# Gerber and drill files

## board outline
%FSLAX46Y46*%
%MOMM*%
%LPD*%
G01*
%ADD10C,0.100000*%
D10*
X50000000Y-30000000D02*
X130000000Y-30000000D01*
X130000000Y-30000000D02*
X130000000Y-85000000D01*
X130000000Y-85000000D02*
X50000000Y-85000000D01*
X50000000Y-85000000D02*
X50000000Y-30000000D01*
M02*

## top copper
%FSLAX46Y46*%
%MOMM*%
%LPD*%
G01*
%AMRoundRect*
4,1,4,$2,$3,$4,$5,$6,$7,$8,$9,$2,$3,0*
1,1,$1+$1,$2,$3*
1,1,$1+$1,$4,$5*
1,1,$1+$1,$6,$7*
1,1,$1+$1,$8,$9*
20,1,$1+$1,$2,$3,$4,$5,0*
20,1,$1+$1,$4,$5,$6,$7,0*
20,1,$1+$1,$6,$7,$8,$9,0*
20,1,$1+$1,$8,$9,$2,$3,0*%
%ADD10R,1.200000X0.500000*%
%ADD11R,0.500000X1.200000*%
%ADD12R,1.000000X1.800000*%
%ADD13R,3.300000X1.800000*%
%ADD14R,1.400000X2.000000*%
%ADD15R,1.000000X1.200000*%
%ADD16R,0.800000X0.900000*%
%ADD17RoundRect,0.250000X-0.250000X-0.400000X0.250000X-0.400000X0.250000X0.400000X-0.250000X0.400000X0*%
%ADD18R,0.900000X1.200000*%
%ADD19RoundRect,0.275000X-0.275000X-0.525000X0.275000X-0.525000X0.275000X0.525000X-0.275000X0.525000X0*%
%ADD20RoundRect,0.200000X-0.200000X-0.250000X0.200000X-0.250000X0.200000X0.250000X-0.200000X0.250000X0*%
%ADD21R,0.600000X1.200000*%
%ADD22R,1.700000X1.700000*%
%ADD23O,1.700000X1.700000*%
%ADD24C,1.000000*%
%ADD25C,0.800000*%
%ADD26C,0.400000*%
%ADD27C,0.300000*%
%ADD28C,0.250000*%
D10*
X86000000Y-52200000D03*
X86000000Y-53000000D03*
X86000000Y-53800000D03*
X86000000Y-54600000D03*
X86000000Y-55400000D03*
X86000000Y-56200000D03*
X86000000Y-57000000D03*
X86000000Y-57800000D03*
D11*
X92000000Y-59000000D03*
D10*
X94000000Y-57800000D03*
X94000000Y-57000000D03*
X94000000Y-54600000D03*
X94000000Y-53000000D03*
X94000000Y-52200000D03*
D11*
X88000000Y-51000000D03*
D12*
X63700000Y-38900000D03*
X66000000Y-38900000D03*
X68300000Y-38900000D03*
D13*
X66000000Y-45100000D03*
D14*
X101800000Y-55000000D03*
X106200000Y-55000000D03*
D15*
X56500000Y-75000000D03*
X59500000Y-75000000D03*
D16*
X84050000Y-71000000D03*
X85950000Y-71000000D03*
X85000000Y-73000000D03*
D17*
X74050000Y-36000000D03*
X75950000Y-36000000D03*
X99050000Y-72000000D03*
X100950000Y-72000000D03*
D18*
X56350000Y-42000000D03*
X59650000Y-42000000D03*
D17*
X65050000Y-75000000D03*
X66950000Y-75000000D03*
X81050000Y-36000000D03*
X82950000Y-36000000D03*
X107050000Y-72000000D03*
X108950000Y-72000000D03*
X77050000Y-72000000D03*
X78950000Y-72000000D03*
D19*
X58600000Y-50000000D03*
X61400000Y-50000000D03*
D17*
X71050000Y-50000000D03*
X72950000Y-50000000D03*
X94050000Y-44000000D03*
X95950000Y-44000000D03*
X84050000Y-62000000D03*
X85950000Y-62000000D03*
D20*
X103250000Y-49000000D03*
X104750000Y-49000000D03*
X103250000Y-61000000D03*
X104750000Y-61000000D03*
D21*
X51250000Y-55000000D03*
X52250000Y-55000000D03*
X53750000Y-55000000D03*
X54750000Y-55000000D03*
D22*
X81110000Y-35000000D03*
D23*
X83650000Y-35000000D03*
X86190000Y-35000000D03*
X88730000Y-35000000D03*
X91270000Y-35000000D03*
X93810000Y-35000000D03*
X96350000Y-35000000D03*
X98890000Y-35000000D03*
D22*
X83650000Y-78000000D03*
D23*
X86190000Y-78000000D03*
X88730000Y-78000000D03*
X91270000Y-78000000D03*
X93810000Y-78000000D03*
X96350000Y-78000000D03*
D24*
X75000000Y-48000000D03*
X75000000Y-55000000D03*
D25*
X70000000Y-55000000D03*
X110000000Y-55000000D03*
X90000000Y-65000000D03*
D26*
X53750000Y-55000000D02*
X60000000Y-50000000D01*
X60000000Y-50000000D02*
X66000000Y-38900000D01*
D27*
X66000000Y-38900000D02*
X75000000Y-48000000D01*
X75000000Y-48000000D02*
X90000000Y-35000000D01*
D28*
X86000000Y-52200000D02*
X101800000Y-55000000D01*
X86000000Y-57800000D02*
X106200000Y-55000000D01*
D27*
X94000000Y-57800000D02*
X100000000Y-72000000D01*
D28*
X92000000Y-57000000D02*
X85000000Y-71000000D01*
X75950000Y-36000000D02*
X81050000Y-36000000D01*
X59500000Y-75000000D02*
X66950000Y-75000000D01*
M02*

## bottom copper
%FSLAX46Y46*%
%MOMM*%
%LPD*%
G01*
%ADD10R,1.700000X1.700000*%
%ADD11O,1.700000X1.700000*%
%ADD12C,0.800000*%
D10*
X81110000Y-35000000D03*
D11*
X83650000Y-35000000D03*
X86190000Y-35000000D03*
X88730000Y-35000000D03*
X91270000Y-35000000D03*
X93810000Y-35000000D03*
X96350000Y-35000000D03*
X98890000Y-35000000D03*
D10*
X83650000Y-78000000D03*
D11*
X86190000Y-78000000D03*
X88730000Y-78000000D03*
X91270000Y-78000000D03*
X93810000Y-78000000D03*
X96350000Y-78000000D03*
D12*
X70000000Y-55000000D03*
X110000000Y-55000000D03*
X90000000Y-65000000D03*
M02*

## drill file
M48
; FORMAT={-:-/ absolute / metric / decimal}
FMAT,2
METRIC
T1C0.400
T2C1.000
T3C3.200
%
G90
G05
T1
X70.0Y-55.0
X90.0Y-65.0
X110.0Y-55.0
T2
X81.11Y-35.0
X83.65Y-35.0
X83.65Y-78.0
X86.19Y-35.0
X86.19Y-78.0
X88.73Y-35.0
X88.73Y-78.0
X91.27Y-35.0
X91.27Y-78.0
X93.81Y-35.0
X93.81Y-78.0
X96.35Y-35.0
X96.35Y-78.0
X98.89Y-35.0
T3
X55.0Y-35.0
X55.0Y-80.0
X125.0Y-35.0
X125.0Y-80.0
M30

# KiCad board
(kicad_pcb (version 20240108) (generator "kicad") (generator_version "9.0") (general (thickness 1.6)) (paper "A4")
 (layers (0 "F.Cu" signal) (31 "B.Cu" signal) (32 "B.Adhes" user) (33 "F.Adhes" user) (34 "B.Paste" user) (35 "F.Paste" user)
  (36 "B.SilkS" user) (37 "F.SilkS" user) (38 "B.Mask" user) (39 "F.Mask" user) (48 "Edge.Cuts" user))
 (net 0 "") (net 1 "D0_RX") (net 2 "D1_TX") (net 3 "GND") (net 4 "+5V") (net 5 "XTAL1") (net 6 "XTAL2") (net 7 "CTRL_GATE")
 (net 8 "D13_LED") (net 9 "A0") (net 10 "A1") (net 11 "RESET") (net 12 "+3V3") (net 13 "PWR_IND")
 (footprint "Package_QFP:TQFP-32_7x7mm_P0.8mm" (layer "F.Cu") (at 90.0 55.0) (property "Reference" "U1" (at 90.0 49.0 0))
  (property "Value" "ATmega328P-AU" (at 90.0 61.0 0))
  (pad "1" smd rect (at -4.0 -2.8) (size 1.2 0.5) (layers "F.Cu" "F.Mask") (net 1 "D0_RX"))
  (pad "2" smd rect (at -4.0 -2.0) (size 1.2 0.5) (layers "F.Cu" "F.Mask") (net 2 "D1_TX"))
  (pad "3" smd rect (at -4.0 -1.2) (size 1.2 0.5) (layers "F.Cu" "F.Mask") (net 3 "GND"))
  (pad "4" smd rect (at -4.0 -0.4) (size 1.2 0.5) (layers "F.Cu" "F.Mask") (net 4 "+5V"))
  (pad "5" smd rect (at -4.0 0.4) (size 1.2 0.5) (layers "F.Cu" "F.Mask") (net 3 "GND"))
  (pad "6" smd rect (at -4.0 1.2) (size 1.2 0.5) (layers "F.Cu" "F.Mask") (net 4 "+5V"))
  (pad "7" smd rect (at -4.0 2.0) (size 1.2 0.5) (layers "F.Cu" "F.Mask") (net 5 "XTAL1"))
  (pad "8" smd rect (at -4.0 2.8) (size 1.2 0.5) (layers "F.Cu" "F.Mask") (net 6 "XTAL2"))
  (pad "15" smd rect (at 2.0 4.0) (size 0.5 1.2) (layers "F.Cu" "F.Mask") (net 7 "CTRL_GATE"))
  (pad "17" smd rect (at 4.0 2.8) (size 1.2 0.5) (layers "F.Cu" "F.Mask") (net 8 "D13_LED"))
  (pad "18" smd rect (at 4.0 2.0) (size 1.2 0.5) (layers "F.Cu" "F.Mask") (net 4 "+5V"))
  (pad "21" smd rect (at 4.0 -0.4) (size 1.2 0.5) (layers "F.Cu" "F.Mask") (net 3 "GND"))
  (pad "23" smd rect (at 4.0 -2.0) (size 1.2 0.5) (layers "F.Cu" "F.Mask") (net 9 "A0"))
  (pad "24" smd rect (at 4.0 -2.8) (size 1.2 0.5) (layers "F.Cu" "F.Mask") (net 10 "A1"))
  (pad "29" smd rect (at -2.0 -4.0) (size 0.5 1.2) (layers "F.Cu" "F.Mask") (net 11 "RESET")))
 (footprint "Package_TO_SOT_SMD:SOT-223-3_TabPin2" (layer "F.Cu") (at 66.0 42.0) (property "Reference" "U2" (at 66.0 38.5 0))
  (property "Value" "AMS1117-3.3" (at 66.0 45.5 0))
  (pad "1" smd rect (at -2.3 -3.1) (size 1.0 1.8) (layers "F.Cu" "F.Mask") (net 3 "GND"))
  (pad "2" smd rect (at 0.0 -3.1) (size 1.0 1.8) (layers "F.Cu" "F.Mask") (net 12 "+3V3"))
  (pad "3" smd rect (at 2.3 -3.1) (size 1.0 1.8) (layers "F.Cu" "F.Mask") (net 4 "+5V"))
  (pad "4" smd rect (at 0.0 3.1) (size 3.3 1.8) (layers "F.Cu" "F.Mask") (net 12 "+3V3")))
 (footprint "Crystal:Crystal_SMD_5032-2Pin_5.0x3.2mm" (layer "F.Cu") (at 104.0 55.0) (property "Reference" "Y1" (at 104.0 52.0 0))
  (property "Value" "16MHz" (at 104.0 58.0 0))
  (pad "1" smd rect (at -2.2 0) (size 1.4 2.0) (layers "F.Cu" "F.Mask") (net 5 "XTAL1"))
  (pad "2" smd rect (at 2.2 0) (size 1.4 2.0) (layers "F.Cu" "F.Mask") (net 6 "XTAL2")))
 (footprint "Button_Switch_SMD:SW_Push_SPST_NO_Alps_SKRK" (layer "F.Cu") (at 58.0 75.0) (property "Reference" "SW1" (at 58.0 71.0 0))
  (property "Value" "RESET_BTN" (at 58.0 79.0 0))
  (pad "1" smd rect (at -1.5 0) (size 1.0 1.2) (layers "F.Cu" "F.Mask") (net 11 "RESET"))
  (pad "2" smd rect (at 1.5 0) (size 1.0 1.2) (layers "F.Cu" "F.Mask") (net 3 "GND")))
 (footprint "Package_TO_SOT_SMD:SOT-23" (layer "F.Cu") (at 85.0 72.0) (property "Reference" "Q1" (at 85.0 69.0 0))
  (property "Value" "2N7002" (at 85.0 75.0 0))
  (pad "1" smd rect (at -0.95 -1.0) (size 0.8 0.9) (layers "F.Cu" "F.Mask") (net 7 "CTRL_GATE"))
  (pad "2" smd rect (at 0.95 -1.0) (size 0.8 0.9) (layers "F.Cu" "F.Mask") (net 3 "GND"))
  (pad "3" smd rect (at 0.0 1.0) (size 0.8 0.9) (layers "F.Cu" "F.Mask") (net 8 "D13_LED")))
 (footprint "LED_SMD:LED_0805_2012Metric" (layer "F.Cu") (at 75.0 36.0) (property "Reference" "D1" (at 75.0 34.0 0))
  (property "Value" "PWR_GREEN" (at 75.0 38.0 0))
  (pad "1" smd roundrect (at -0.95 0) (size 1.0 1.3) (layers "F.Cu" "F.Mask") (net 3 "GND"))
  (pad "2" smd roundrect (at 0.95 0) (size 1.0 1.3) (layers "F.Cu" "F.Mask") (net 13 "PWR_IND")))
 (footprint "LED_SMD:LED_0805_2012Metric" (layer "F.Cu") (at 100.0 72.0) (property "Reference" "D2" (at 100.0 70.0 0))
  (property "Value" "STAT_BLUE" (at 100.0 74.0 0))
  (pad "1" smd roundrect (at -0.95 0) (size 1.0 1.3) (layers "F.Cu" "F.Mask") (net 3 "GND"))
  (pad "2" smd roundrect (at 0.95 0) (size 1.0 1.3) (layers "F.Cu" "F.Mask") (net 8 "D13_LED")))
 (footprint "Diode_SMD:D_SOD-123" (layer "F.Cu") (at 58.0 42.0) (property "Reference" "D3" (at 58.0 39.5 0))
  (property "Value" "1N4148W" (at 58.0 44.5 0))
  (pad "1" smd rect (at -1.65 0) (size 0.9 1.2) (layers "F.Cu" "F.Mask") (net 4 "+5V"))
  (pad "2" smd rect (at 1.65 0) (size 0.9 1.2) (layers "F.Cu" "F.Mask") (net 4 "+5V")))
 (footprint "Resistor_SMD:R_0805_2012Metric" (layer "F.Cu") (at 66.0 75.0) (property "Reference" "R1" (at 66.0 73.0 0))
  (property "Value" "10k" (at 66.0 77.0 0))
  (pad "1" smd roundrect (at -0.95 0) (size 1.0 1.3) (layers "F.Cu" "F.Mask") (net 4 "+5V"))
  (pad "2" smd roundrect (at 0.95 0) (size 1.0 1.3) (layers "F.Cu" "F.Mask") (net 11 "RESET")))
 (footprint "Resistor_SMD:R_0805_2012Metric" (layer "F.Cu") (at 82.0 36.0) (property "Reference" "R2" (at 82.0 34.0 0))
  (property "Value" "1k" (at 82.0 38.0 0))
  (pad "1" smd roundrect (at -0.95 0) (size 1.0 1.3) (layers "F.Cu" "F.Mask") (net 4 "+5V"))
  (pad "2" smd roundrect (at 0.95 0) (size 1.0 1.3) (layers "F.Cu" "F.Mask") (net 13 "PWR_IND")))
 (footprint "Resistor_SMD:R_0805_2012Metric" (layer "F.Cu") (at 108.0 72.0) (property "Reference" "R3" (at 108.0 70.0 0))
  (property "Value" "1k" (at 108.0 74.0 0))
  (pad "1" smd roundrect (at -0.95 0) (size 1.0 1.3) (layers "F.Cu" "F.Mask") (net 8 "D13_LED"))
  (pad "2" smd roundrect (at 0.95 0) (size 1.0 1.3) (layers "F.Cu" "F.Mask") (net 4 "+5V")))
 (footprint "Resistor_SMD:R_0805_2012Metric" (layer "F.Cu") (at 78.0 72.0) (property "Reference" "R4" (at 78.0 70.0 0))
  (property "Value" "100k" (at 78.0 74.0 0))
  (pad "1" smd roundrect (at -0.95 0) (size 1.0 1.3) (layers "F.Cu" "F.Mask") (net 7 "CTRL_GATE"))
  (pad "2" smd roundrect (at 0.95 0) (size 1.0 1.3) (layers "F.Cu" "F.Mask") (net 3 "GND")))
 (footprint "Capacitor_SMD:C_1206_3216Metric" (layer "F.Cu") (at 60.0 50.0) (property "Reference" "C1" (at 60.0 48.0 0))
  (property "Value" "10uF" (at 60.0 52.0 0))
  (pad "1" smd roundrect (at -1.4 0) (size 1.1 1.6) (layers "F.Cu" "F.Mask") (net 4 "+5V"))
  (pad "2" smd roundrect (at 1.4 0) (size 1.1 1.6) (layers "F.Cu" "F.Mask") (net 3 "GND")))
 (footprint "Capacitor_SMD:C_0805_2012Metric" (layer "F.Cu") (at 72.0 50.0) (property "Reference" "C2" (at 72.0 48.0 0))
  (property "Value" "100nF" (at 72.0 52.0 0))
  (pad "1" smd roundrect (at -0.95 0) (size 1.0 1.3) (layers "F.Cu" "F.Mask") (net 12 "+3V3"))
  (pad "2" smd roundrect (at 0.95 0) (size 1.0 1.3) (layers "F.Cu" "F.Mask") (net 3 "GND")))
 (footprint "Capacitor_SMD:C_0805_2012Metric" (layer "F.Cu") (at 95.0 44.0) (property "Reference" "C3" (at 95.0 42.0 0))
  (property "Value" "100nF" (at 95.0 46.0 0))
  (pad "1" smd roundrect (at -0.95 0) (size 1.0 1.3) (layers "F.Cu" "F.Mask") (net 4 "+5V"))
  (pad "2" smd roundrect (at 0.95 0) (size 1.0 1.3) (layers "F.Cu" "F.Mask") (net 3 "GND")))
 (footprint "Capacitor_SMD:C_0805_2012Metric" (layer "F.Cu") (at 85.0 62.0) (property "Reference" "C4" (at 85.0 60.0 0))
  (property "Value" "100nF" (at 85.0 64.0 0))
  (pad "1" smd roundrect (at -0.95 0) (size 1.0 1.3) (layers "F.Cu" "F.Mask") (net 4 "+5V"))
  (pad "2" smd roundrect (at 0.95 0) (size 1.0 1.3) (layers "F.Cu" "F.Mask") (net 3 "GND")))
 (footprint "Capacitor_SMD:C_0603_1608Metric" (layer "F.Cu") (at 104.0 49.0) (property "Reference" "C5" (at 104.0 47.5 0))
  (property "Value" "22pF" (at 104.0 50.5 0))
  (pad "1" smd roundrect (at -0.75 0) (size 0.8 0.9) (layers "F.Cu" "F.Mask") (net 5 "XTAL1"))
  (pad "2" smd roundrect (at 0.75 0) (size 0.8 0.9) (layers "F.Cu" "F.Mask") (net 3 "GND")))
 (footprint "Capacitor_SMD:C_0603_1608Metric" (layer "F.Cu") (at 104.0 61.0) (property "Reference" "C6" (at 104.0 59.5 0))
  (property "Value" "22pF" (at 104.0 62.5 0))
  (pad "1" smd roundrect (at -0.75 0) (size 0.8 0.9) (layers "F.Cu" "F.Mask") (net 6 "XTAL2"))
  (pad "2" smd roundrect (at 0.75 0) (size 0.8 0.9) (layers "F.Cu" "F.Mask") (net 3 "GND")))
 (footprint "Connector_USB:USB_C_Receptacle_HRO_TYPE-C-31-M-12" (layer "F.Cu") (at 53.0 58.0) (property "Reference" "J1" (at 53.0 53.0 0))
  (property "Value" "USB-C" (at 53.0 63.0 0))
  (pad "A1" smd rect (at -1.75 -3.0) (size 0.6 1.2) (layers "F.Cu" "F.Mask") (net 3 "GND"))
  (pad "A4" smd rect (at -0.75 -3.0) (size 0.6 1.2) (layers "F.Cu" "F.Mask") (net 4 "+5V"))
  (pad "B4" smd rect (at 0.75 -3.0) (size 0.6 1.2) (layers "F.Cu" "F.Mask") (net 4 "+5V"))
  (pad "B1" smd rect (at 1.75 -3.0) (size 0.6 1.2) (layers "F.Cu" "F.Mask") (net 3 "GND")))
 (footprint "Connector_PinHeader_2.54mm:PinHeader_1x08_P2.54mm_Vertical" (layer "F.Cu") (at 90.0 35.0)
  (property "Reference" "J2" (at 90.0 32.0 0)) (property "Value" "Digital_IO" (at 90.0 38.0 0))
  (pad "1" thru_hole rect (at -8.89 0) (size 1.7 1.7) (drill 1.0) (layers "*.Cu" "*.Mask") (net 1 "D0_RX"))
  (pad "2" thru_hole oval (at -6.35 0) (size 1.7 1.7) (drill 1.0) (layers "*.Cu" "*.Mask") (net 2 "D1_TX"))
  (pad "3" thru_hole oval (at -3.81 0) (size 1.7 1.7) (drill 1.0) (layers "*.Cu" "*.Mask") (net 3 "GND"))
  (pad "4" thru_hole oval (at -1.27 0) (size 1.7 1.7) (drill 1.0) (layers "*.Cu" "*.Mask") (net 4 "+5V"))
  (pad "5" thru_hole oval (at 1.27 0) (size 1.7 1.7) (drill 1.0) (layers "*.Cu" "*.Mask") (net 12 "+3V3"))
  (pad "6" thru_hole oval (at 3.81 0) (size 1.7 1.7) (drill 1.0) (layers "*.Cu" "*.Mask") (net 11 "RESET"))
  (pad "7" thru_hole oval (at 6.35 0) (size 1.7 1.7) (drill 1.0) (layers "*.Cu" "*.Mask") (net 7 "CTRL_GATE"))
  (pad "8" thru_hole oval (at 8.89 0) (size 1.7 1.7) (drill 1.0) (layers "*.Cu" "*.Mask") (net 8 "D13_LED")))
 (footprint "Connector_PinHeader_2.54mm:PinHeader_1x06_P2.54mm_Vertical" (layer "F.Cu") (at 90.0 78.0)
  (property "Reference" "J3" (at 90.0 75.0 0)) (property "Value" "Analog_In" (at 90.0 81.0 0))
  (pad "1" thru_hole rect (at -6.35 0) (size 1.7 1.7) (drill 1.0) (layers "*.Cu" "*.Mask") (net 9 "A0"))
  (pad "2" thru_hole oval (at -3.81 0) (size 1.7 1.7) (drill 1.0) (layers "*.Cu" "*.Mask") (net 10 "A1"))
  (pad "3" thru_hole oval (at -1.27 0) (size 1.7 1.7) (drill 1.0) (layers "*.Cu" "*.Mask") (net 3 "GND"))
  (pad "4" thru_hole oval (at 1.27 0) (size 1.7 1.7) (drill 1.0) (layers "*.Cu" "*.Mask") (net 3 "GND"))
  (pad "5" thru_hole oval (at 3.81 0) (size 1.7 1.7) (drill 1.0) (layers "*.Cu" "*.Mask") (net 4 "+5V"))
  (pad "6" thru_hole oval (at 6.35 0) (size 1.7 1.7) (drill 1.0) (layers "*.Cu" "*.Mask") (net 12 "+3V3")))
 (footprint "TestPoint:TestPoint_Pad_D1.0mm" (layer "F.Cu") (at 75.0 48.0) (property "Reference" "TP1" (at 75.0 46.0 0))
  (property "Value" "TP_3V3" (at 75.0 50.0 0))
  (pad "1" smd circle (at 0 0) (size 1.0 1.0) (layers "F.Cu" "F.Mask") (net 12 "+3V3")))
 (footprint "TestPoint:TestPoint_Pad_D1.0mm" (layer "F.Cu") (at 75.0 55.0) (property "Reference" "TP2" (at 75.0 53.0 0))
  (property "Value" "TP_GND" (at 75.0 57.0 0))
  (pad "1" smd circle (at 0 0) (size 1.0 1.0) (layers "F.Cu" "F.Mask") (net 3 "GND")))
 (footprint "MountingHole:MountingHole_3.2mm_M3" (layer "F.Cu") (at 55.0 35.0) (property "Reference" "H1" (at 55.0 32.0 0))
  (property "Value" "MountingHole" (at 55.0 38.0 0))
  (pad "" np_thru_hole circle (at 0 0) (size 3.2 3.2) (drill 3.2) (layers "*.Cu" "*.Mask")))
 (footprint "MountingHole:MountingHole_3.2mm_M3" (layer "F.Cu") (at 125.0 35.0) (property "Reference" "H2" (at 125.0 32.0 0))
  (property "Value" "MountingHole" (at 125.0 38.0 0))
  (pad "" np_thru_hole circle (at 0 0) (size 3.2 3.2) (drill 3.2) (layers "*.Cu" "*.Mask")))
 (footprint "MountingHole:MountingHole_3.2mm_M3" (layer "F.Cu") (at 55.0 80.0) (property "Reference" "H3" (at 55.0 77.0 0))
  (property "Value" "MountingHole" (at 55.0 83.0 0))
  (pad "" np_thru_hole circle (at 0 0) (size 3.2 3.2) (drill 3.2) (layers "*.Cu" "*.Mask")))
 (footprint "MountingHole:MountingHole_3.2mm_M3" (layer "F.Cu") (at 125.0 80.0) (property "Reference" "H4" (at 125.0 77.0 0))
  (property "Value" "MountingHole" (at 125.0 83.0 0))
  (pad "" np_thru_hole circle (at 0 0) (size 3.2 3.2) (drill 3.2) (layers "*.Cu" "*.Mask")))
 (segment (start 53.75 55.0) (end 60.0 50.0) (width 0.4) (layer "F.Cu") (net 4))
 (segment (start 60.0 50.0) (end 66.0 38.9) (width 0.4) (layer "F.Cu") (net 4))
 (segment (start 66.0 38.9) (end 75.0 48.0) (width 0.3) (layer "F.Cu") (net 12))
 (segment (start 75.0 48.0) (end 90.0 35.0) (width 0.3) (layer "F.Cu") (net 12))
 (segment (start 86.0 52.2) (end 101.8 55.0) (width 0.25) (layer "F.Cu") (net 5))
 (segment (start 86.0 57.8) (end 106.2 55.0) (width 0.25) (layer "F.Cu") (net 6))
 (segment (start 94.0 57.8) (end 100.0 72.0) (width 0.3) (layer "F.Cu") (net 8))
 (segment (start 92.0 57.0) (end 85.0 71.0) (width 0.25) (layer "F.Cu") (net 7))
 (segment (start 75.95 36.0) (end 81.05 36.0) (width 0.25) (layer "F.Cu") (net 13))
 (segment (start 59.5 75.0) (end 66.95 75.0) (width 0.25) (layer "F.Cu") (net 11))
 (via (at 70.0 55.0) (size 0.8) (drill 0.4) (layers "F.Cu" "B.Cu") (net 3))
 (via (at 110.0 55.0) (size 0.8) (drill 0.4) (layers "F.Cu" "B.Cu") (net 3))
 (via (at 90.0 65.0) (size 0.8) (drill 0.4) (layers "F.Cu" "B.Cu") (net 4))
 (gr_line (start 50.0 30.0) (end 130.0 30.0) (layer "Edge.Cuts") (width 0.1))
 (gr_line (start 130.0 30.0) (end 130.0 85.0) (layer "Edge.Cuts") (width 0.1))
 (gr_line (start 130.0 85.0) (end 50.0 85.0) (layer "Edge.Cuts") (width 0.1))
 (gr_line (start 50.0 85.0) (end 50.0 30.0) (layer "Edge.Cuts") (width 0.1)))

